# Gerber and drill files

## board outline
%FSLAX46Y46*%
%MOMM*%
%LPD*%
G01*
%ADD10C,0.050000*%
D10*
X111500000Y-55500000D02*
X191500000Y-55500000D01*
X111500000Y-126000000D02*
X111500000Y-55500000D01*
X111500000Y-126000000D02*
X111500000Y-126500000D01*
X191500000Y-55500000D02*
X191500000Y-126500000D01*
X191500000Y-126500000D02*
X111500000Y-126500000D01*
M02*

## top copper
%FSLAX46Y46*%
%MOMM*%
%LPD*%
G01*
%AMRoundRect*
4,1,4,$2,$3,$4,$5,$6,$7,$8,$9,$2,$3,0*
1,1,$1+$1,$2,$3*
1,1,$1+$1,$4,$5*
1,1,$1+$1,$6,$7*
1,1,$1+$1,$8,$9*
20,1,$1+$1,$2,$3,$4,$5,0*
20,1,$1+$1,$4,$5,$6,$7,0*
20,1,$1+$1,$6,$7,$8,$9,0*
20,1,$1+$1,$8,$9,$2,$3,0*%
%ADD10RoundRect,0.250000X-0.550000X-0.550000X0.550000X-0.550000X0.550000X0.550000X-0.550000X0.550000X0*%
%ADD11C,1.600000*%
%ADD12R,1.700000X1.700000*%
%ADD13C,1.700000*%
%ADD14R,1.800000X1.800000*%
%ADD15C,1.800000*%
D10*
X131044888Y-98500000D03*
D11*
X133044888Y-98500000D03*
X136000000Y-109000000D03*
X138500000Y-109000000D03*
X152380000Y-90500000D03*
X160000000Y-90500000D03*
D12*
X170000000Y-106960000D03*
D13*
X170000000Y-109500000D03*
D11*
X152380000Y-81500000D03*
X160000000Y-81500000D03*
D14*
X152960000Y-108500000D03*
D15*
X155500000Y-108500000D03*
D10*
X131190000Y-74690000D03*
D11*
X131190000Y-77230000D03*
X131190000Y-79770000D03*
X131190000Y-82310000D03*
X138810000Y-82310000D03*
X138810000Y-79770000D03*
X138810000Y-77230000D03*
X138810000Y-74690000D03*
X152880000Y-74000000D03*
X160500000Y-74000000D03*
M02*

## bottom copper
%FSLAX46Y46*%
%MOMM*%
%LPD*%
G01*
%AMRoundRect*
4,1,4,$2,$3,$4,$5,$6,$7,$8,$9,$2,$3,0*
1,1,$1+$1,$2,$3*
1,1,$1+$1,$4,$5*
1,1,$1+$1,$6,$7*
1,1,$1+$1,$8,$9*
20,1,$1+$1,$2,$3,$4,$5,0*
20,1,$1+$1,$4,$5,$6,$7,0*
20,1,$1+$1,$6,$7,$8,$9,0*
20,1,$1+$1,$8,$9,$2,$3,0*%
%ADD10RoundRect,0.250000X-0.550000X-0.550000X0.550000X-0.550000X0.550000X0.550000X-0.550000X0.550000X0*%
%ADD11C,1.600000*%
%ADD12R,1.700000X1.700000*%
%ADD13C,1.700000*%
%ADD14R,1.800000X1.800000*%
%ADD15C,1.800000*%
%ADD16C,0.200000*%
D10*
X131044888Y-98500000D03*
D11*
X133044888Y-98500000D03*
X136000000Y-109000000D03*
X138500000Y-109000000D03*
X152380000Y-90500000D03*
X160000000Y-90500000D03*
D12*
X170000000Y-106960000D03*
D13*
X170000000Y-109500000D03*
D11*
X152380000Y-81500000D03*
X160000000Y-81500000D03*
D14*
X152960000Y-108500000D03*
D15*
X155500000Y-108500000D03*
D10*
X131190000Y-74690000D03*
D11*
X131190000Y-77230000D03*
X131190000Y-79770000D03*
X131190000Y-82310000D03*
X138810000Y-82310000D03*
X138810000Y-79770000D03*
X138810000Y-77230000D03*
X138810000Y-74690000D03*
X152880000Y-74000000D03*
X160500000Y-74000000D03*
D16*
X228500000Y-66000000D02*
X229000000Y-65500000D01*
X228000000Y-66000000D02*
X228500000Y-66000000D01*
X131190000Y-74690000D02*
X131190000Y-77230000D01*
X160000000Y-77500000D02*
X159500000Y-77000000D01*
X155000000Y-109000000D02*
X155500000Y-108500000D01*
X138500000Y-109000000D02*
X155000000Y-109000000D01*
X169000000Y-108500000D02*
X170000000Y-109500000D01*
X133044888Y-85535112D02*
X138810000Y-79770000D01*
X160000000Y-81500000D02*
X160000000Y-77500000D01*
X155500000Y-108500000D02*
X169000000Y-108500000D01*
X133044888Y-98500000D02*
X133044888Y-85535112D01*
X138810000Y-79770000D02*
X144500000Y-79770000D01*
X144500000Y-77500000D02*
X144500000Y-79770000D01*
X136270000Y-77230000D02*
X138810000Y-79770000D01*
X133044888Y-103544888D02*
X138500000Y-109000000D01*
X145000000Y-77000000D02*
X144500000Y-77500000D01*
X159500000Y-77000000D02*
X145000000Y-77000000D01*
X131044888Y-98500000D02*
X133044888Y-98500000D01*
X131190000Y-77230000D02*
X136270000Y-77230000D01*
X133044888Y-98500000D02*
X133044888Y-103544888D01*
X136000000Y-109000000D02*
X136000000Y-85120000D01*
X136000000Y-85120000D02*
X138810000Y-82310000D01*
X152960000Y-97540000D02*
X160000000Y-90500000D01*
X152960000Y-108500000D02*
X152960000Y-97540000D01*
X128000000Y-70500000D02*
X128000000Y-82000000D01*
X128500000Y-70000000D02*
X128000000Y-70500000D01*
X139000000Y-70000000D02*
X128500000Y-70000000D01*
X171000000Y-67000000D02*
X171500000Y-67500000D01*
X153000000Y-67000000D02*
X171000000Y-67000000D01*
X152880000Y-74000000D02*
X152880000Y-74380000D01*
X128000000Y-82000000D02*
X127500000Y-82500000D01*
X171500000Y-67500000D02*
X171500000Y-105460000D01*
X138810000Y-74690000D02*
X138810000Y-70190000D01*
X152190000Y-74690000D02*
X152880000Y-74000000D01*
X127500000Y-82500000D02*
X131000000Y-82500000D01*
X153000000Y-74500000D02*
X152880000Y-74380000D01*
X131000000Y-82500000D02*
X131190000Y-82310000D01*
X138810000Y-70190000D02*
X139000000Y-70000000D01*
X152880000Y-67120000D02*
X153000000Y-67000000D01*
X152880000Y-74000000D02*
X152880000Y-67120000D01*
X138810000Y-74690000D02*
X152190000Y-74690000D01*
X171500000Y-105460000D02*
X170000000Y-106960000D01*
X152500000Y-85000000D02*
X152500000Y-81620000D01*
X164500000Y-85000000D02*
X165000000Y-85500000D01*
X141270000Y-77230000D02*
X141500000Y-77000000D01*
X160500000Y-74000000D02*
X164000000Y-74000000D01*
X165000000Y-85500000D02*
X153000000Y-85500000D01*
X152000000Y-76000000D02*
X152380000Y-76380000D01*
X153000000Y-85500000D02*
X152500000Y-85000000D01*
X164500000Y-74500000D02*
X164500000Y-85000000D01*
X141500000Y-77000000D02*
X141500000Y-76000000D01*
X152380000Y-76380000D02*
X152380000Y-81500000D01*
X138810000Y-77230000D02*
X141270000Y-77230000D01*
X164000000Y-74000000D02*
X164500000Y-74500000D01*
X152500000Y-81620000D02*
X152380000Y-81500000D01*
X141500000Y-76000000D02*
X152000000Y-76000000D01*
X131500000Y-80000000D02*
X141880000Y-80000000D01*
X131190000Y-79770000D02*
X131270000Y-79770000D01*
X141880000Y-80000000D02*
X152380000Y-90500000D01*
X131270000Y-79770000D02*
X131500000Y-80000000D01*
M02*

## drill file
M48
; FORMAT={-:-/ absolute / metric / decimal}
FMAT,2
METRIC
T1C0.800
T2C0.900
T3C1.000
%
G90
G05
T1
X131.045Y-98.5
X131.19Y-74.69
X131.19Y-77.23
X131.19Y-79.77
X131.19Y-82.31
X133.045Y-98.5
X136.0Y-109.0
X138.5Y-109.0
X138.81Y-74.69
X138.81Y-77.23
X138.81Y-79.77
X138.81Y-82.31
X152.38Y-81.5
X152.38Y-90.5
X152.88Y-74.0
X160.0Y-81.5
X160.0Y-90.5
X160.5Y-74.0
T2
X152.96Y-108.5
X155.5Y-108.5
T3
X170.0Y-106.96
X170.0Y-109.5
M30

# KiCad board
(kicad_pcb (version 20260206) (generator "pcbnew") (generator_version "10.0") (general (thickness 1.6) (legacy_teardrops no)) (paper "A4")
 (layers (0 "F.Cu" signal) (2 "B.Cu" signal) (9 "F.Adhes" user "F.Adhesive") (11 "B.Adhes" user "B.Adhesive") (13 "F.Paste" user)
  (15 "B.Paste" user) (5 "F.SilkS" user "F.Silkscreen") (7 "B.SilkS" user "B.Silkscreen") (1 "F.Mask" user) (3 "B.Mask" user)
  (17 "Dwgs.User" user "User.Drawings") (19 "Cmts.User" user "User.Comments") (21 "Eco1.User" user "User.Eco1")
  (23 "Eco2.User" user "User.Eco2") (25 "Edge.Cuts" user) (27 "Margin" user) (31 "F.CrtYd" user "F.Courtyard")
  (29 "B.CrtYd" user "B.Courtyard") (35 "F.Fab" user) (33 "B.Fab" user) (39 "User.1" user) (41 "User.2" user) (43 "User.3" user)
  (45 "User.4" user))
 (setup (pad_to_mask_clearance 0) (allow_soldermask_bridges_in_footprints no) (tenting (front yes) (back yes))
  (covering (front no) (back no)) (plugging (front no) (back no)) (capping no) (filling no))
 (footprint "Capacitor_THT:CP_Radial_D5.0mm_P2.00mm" (layer "F.Cu") (at 131.044888 98.5)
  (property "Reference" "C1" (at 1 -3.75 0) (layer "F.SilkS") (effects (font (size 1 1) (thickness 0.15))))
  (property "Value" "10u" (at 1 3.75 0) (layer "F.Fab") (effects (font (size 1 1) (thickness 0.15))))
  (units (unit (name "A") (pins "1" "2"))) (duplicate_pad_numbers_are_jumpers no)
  (pad "1" thru_hole roundrect (at 0 0) (size 1.6 1.6) (drill 0.8) (layers "*.Cu" "*.Mask") (remove_unused_layers no)
   (roundrect_rratio 0.15625) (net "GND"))
  (pad "2" thru_hole circle (at 2 0) (size 1.6 1.6) (drill 0.8) (layers "*.Cu" "*.Mask") (remove_unused_layers no) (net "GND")))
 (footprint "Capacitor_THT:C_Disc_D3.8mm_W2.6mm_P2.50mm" (layer "F.Cu") (at 136 109)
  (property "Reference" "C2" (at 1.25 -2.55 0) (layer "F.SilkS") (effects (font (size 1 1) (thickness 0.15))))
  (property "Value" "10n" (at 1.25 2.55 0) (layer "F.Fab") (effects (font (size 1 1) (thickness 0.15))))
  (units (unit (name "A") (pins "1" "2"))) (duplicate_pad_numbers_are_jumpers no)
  (pad "1" thru_hole circle (at 0 0) (size 1.6 1.6) (drill 0.8) (layers "*.Cu" "*.Mask") (remove_unused_layers no) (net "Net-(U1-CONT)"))
  (pad "2" thru_hole circle (at 2.5 0) (size 1.6 1.6) (drill 0.8) (layers "*.Cu" "*.Mask") (remove_unused_layers no) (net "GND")))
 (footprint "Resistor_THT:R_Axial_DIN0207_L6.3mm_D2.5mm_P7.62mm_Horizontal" (layer "F.Cu") (at 152.38 90.5)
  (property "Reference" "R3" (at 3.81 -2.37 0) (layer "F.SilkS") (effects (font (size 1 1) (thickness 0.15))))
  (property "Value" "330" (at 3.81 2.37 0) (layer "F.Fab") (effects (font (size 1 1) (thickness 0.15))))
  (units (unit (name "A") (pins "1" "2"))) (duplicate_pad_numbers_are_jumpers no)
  (pad "1" thru_hole circle (at 0 0) (size 1.6 1.6) (drill 0.8) (layers "*.Cu" "*.Mask") (remove_unused_layers no) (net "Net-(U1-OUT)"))
  (pad "2" thru_hole circle (at 7.62 0) (size 1.6 1.6) (drill 0.8) (layers "*.Cu" "*.Mask") (remove_unused_layers no) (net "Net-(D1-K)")))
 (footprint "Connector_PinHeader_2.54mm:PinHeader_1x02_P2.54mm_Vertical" (layer "F.Cu") (at 170 106.96)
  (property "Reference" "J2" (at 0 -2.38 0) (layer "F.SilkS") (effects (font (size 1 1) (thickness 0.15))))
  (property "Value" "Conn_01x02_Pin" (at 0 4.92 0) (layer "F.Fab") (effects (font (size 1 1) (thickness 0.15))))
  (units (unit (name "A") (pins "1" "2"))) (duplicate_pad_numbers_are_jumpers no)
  (pad "1" thru_hole rect (at 0 0) (size 1.7 1.7) (drill 1) (layers "*.Cu" "*.Mask") (remove_unused_layers no) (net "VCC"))
  (pad "2" thru_hole circle (at 0 2.54) (size 1.7 1.7) (drill 1) (layers "*.Cu" "*.Mask") (remove_unused_layers no) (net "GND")))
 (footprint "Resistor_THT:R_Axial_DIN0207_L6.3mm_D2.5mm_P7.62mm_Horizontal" (layer "F.Cu") (at 152.38 81.5)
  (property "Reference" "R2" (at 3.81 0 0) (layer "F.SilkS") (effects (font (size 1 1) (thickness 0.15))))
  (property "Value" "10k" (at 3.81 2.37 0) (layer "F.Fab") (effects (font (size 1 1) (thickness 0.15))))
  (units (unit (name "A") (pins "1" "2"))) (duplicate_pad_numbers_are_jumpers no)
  (pad "1" thru_hole circle (at 0 0) (size 1.6 1.6) (drill 0.8) (layers "*.Cu" "*.Mask") (remove_unused_layers no) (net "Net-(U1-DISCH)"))
  (pad "2" thru_hole circle (at 7.62 0) (size 1.6 1.6) (drill 0.8) (layers "*.Cu" "*.Mask") (remove_unused_layers no) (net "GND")))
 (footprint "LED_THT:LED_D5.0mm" (layer "F.Cu") (at 152.96 108.5)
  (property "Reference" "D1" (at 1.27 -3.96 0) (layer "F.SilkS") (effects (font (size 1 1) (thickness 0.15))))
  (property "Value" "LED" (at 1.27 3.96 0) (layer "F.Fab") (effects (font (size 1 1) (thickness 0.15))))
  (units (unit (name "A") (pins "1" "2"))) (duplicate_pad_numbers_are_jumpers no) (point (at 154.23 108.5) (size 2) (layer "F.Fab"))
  (pad "1" thru_hole rect (at 0 0) (size 1.8 1.8) (drill 0.9) (layers "*.Cu" "*.Mask") (remove_unused_layers no) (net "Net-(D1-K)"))
  (pad "2" thru_hole circle (at 2.54 0) (size 1.8 1.8) (drill 0.9) (layers "*.Cu" "*.Mask") (remove_unused_layers no) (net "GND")))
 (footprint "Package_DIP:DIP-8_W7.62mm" (layer "F.Cu") (at 131.19 74.69)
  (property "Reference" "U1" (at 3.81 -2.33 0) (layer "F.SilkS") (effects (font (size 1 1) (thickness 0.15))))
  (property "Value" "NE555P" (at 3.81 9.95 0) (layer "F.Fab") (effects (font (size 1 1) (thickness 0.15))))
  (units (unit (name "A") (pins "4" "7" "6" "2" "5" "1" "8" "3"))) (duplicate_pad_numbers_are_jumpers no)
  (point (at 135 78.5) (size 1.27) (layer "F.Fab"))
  (pad "1" thru_hole roundrect (at 0 0) (size 1.6 1.6) (drill 0.8) (layers "*.Cu" "*.Mask") (remove_unused_layers no)
   (roundrect_rratio 0.15625) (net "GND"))
  (pad "2" thru_hole circle (at 0 2.54) (size 1.6 1.6) (drill 0.8) (layers "*.Cu" "*.Mask") (remove_unused_layers no) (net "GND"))
  (pad "3" thru_hole circle (at 0 5.08) (size 1.6 1.6) (drill 0.8) (layers "*.Cu" "*.Mask") (remove_unused_layers no) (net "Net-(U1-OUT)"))
  (pad "4" thru_hole circle (at 0 7.62) (size 1.6 1.6) (drill 0.8) (layers "*.Cu" "*.Mask") (remove_unused_layers no) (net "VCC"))
  (pad "5" thru_hole circle (at 7.62 7.62) (size 1.6 1.6) (drill 0.8) (layers "*.Cu" "*.Mask") (remove_unused_layers no)
   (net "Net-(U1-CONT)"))
  (pad "6" thru_hole circle (at 7.62 5.08) (size 1.6 1.6) (drill 0.8) (layers "*.Cu" "*.Mask") (remove_unused_layers no) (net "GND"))
  (pad "7" thru_hole circle (at 7.62 2.54) (size 1.6 1.6) (drill 0.8) (layers "*.Cu" "*.Mask") (remove_unused_layers no)
   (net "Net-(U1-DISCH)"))
  (pad "8" thru_hole circle (at 7.62 0) (size 1.6 1.6) (drill 0.8) (layers "*.Cu" "*.Mask") (remove_unused_layers no) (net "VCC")))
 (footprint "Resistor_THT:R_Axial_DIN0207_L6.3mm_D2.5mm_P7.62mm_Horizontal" (layer "F.Cu") (at 152.88 74)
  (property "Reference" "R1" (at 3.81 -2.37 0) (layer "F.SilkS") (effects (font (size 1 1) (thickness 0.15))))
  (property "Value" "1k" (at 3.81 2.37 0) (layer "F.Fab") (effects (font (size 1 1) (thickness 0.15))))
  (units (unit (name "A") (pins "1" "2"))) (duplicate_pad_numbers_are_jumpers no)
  (pad "1" thru_hole circle (at 0 0) (size 1.6 1.6) (drill 0.8) (layers "*.Cu" "*.Mask") (remove_unused_layers no) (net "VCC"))
  (pad "2" thru_hole circle (at 7.62 0) (size 1.6 1.6) (drill 0.8) (layers "*.Cu" "*.Mask") (remove_unused_layers no) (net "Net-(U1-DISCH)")))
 (gr_line (start 111.5 55.5) (end 191.5 55.5) (stroke (width 0.05) (type default)) (layer "Edge.Cuts"))
 (gr_line (start 111.5 126) (end 111.5 55.5) (stroke (width 0.05) (type default)) (layer "Edge.Cuts"))
 (gr_line (start 111.5 126) (end 111.5 126.5) (stroke (width 0.05) (type default)) (layer "Edge.Cuts"))
 (gr_line (start 191.5 55.5) (end 191.5 126.5) (stroke (width 0.05) (type default)) (layer "Edge.Cuts"))
 (gr_line (start 191.5 126.5) (end 111.5 126.5) (stroke (width 0.05) (type default)) (layer "Edge.Cuts"))
 (segment (start 228.5 66) (end 229 65.5) (width 0.2) (layer "B.Cu") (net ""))
 (segment (start 228 66) (end 228.5 66) (width 0.2) (layer "B.Cu") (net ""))
 (segment (start 131.19 74.69) (end 131.19 77.23) (width 0.2) (layer "B.Cu") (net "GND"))
 (segment (start 160 77.5) (end 159.5 77) (width 0.2) (layer "B.Cu") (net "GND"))
 (segment (start 155 109) (end 155.5 108.5) (width 0.2) (layer "B.Cu") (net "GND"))
 (segment (start 138.5 109) (end 155 109) (width 0.2) (layer "B.Cu") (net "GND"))
 (segment (start 169 108.5) (end 170 109.5) (width 0.2) (layer "B.Cu") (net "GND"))
 (segment (start 133.044888 85.535112) (end 138.81 79.77) (width 0.2) (layer "B.Cu") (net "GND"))
 (segment (start 160 81.5) (end 160 77.5) (width 0.2) (layer "B.Cu") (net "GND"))
 (segment (start 155.5 108.5) (end 169 108.5) (width 0.2) (layer "B.Cu") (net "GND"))
 (segment (start 133.044888 98.5) (end 133.044888 85.535112) (width 0.2) (layer "B.Cu") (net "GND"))
 (segment (start 138.81 79.77) (end 144.5 79.77) (width 0.2) (layer "B.Cu") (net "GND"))
 (segment (start 144.5 77.5) (end 144.5 79.77) (width 0.2) (layer "B.Cu") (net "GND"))
 (segment (start 136.27 77.23) (end 138.81 79.77) (width 0.2) (layer "B.Cu") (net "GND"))
 (segment (start 133.044888 103.544888) (end 138.5 109) (width 0.2) (layer "B.Cu") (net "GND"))
 (segment (start 145 77) (end 144.5 77.5) (width 0.2) (layer "B.Cu") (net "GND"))
 (segment (start 159.5 77) (end 145 77) (width 0.2) (layer "B.Cu") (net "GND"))
 (segment (start 131.044888 98.5) (end 133.044888 98.5) (width 0.2) (layer "B.Cu") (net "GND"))
 (segment (start 131.19 77.23) (end 136.27 77.23) (width 0.2) (layer "B.Cu") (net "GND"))
 (segment (start 133.044888 98.5) (end 133.044888 103.544888) (width 0.2) (layer "B.Cu") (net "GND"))
 (segment (start 136 109) (end 136 85.12) (width 0.2) (layer "B.Cu") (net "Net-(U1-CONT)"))
 (segment (start 136 85.12) (end 138.81 82.31) (width 0.2) (layer "B.Cu") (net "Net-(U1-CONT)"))
 (segment (start 152.96 97.54) (end 160 90.5) (width 0.2) (layer "B.Cu") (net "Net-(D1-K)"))
 (segment (start 152.96 108.5) (end 152.96 97.54) (width 0.2) (layer "B.Cu") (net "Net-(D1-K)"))
 (segment (start 128 70.5) (end 128 82) (width 0.2) (layer "B.Cu") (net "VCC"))
 (segment (start 128.5 70) (end 128 70.5) (width 0.2) (layer "B.Cu") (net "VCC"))
 (segment (start 139 70) (end 128.5 70) (width 0.2) (layer "B.Cu") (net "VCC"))
 (segment (start 171 67) (end 171.5 67.5) (width 0.2) (layer "B.Cu") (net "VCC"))
 (segment (start 153 67) (end 171 67) (width 0.2) (layer "B.Cu") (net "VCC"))
 (segment (start 152.88 74) (end 152.88 74.38) (width 0.2) (layer "B.Cu") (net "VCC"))
 (segment (start 128 82) (end 127.5 82.5) (width 0.2) (layer "B.Cu") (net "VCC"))
 (segment (start 171.5 67.5) (end 171.5 105.46) (width 0.2) (layer "B.Cu") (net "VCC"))
 (segment (start 138.81 74.69) (end 138.81 70.19) (width 0.2) (layer "B.Cu") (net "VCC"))
 (segment (start 152.19 74.69) (end 152.88 74) (width 0.2) (layer "B.Cu") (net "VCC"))
 (segment (start 127.5 82.5) (end 131 82.5) (width 0.2) (layer "B.Cu") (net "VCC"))
 (segment (start 153 74.5) (end 152.88 74.38) (width 0.2) (layer "B.Cu") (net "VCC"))
 (segment (start 131 82.5) (end 131.19 82.31) (width 0.2) (layer "B.Cu") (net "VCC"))
 (segment (start 138.81 70.19) (end 139 70) (width 0.2) (layer "B.Cu") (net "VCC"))
 (segment (start 152.88 67.12) (end 153 67) (width 0.2) (layer "B.Cu") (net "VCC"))
 (segment (start 152.88 74) (end 152.88 67.12) (width 0.2) (layer "B.Cu") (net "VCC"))
 (segment (start 138.81 74.69) (end 152.19 74.69) (width 0.2) (layer "B.Cu") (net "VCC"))
 (segment (start 171.5 105.46) (end 170 106.96) (width 0.2) (layer "B.Cu") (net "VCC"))
 (segment (start 152.5 85) (end 152.5 81.62) (width 0.2) (layer "B.Cu") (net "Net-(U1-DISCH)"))
 (segment (start 164.5 85) (end 165 85.5) (width 0.2) (layer "B.Cu") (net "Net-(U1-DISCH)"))
 (segment (start 141.27 77.23) (end 141.5 77) (width 0.2) (layer "B.Cu") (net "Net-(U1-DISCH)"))
 (segment (start 160.5 74) (end 164 74) (width 0.2) (layer "B.Cu") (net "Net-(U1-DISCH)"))
 (segment (start 165 85.5) (end 153 85.5) (width 0.2) (layer "B.Cu") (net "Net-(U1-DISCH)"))
 (segment (start 152 76) (end 152.38 76.38) (width 0.2) (layer "B.Cu") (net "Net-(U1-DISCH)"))
 (segment (start 153 85.5) (end 152.5 85) (width 0.2) (layer "B.Cu") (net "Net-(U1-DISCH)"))
 (segment (start 164.5 74.5) (end 164.5 85) (width 0.2) (layer "B.Cu") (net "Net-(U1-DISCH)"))
 (segment (start 141.5 77) (end 141.5 76) (width 0.2) (layer "B.Cu") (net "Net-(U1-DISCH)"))
 (segment (start 152.38 76.38) (end 152.38 81.5) (width 0.2) (layer "B.Cu") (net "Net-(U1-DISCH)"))
 (segment (start 138.81 77.23) (end 141.27 77.23) (width 0.2) (layer "B.Cu") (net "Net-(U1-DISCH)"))
 (segment (start 164 74) (end 164.5 74.5) (width 0.2) (layer "B.Cu") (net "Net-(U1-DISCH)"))
 (segment (start 152.5 81.62) (end 152.38 81.5) (width 0.2) (layer "B.Cu") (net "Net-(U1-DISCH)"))
 (segment (start 141.5 76) (end 152 76) (width 0.2) (layer "B.Cu") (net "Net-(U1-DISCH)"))
 (segment (start 131.5 80) (end 141.88 80) (width 0.2) (layer "B.Cu") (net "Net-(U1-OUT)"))
 (segment (start 131.19 79.77) (end 131.27 79.77) (width 0.2) (layer "B.Cu") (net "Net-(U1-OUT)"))
 (segment (start 141.88 80) (end 152.38 90.5) (width 0.2) (layer "B.Cu") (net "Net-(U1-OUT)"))
 (segment (start 131.27 79.77) (end 131.5 80) (width 0.2) (layer "B.Cu") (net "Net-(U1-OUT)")))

